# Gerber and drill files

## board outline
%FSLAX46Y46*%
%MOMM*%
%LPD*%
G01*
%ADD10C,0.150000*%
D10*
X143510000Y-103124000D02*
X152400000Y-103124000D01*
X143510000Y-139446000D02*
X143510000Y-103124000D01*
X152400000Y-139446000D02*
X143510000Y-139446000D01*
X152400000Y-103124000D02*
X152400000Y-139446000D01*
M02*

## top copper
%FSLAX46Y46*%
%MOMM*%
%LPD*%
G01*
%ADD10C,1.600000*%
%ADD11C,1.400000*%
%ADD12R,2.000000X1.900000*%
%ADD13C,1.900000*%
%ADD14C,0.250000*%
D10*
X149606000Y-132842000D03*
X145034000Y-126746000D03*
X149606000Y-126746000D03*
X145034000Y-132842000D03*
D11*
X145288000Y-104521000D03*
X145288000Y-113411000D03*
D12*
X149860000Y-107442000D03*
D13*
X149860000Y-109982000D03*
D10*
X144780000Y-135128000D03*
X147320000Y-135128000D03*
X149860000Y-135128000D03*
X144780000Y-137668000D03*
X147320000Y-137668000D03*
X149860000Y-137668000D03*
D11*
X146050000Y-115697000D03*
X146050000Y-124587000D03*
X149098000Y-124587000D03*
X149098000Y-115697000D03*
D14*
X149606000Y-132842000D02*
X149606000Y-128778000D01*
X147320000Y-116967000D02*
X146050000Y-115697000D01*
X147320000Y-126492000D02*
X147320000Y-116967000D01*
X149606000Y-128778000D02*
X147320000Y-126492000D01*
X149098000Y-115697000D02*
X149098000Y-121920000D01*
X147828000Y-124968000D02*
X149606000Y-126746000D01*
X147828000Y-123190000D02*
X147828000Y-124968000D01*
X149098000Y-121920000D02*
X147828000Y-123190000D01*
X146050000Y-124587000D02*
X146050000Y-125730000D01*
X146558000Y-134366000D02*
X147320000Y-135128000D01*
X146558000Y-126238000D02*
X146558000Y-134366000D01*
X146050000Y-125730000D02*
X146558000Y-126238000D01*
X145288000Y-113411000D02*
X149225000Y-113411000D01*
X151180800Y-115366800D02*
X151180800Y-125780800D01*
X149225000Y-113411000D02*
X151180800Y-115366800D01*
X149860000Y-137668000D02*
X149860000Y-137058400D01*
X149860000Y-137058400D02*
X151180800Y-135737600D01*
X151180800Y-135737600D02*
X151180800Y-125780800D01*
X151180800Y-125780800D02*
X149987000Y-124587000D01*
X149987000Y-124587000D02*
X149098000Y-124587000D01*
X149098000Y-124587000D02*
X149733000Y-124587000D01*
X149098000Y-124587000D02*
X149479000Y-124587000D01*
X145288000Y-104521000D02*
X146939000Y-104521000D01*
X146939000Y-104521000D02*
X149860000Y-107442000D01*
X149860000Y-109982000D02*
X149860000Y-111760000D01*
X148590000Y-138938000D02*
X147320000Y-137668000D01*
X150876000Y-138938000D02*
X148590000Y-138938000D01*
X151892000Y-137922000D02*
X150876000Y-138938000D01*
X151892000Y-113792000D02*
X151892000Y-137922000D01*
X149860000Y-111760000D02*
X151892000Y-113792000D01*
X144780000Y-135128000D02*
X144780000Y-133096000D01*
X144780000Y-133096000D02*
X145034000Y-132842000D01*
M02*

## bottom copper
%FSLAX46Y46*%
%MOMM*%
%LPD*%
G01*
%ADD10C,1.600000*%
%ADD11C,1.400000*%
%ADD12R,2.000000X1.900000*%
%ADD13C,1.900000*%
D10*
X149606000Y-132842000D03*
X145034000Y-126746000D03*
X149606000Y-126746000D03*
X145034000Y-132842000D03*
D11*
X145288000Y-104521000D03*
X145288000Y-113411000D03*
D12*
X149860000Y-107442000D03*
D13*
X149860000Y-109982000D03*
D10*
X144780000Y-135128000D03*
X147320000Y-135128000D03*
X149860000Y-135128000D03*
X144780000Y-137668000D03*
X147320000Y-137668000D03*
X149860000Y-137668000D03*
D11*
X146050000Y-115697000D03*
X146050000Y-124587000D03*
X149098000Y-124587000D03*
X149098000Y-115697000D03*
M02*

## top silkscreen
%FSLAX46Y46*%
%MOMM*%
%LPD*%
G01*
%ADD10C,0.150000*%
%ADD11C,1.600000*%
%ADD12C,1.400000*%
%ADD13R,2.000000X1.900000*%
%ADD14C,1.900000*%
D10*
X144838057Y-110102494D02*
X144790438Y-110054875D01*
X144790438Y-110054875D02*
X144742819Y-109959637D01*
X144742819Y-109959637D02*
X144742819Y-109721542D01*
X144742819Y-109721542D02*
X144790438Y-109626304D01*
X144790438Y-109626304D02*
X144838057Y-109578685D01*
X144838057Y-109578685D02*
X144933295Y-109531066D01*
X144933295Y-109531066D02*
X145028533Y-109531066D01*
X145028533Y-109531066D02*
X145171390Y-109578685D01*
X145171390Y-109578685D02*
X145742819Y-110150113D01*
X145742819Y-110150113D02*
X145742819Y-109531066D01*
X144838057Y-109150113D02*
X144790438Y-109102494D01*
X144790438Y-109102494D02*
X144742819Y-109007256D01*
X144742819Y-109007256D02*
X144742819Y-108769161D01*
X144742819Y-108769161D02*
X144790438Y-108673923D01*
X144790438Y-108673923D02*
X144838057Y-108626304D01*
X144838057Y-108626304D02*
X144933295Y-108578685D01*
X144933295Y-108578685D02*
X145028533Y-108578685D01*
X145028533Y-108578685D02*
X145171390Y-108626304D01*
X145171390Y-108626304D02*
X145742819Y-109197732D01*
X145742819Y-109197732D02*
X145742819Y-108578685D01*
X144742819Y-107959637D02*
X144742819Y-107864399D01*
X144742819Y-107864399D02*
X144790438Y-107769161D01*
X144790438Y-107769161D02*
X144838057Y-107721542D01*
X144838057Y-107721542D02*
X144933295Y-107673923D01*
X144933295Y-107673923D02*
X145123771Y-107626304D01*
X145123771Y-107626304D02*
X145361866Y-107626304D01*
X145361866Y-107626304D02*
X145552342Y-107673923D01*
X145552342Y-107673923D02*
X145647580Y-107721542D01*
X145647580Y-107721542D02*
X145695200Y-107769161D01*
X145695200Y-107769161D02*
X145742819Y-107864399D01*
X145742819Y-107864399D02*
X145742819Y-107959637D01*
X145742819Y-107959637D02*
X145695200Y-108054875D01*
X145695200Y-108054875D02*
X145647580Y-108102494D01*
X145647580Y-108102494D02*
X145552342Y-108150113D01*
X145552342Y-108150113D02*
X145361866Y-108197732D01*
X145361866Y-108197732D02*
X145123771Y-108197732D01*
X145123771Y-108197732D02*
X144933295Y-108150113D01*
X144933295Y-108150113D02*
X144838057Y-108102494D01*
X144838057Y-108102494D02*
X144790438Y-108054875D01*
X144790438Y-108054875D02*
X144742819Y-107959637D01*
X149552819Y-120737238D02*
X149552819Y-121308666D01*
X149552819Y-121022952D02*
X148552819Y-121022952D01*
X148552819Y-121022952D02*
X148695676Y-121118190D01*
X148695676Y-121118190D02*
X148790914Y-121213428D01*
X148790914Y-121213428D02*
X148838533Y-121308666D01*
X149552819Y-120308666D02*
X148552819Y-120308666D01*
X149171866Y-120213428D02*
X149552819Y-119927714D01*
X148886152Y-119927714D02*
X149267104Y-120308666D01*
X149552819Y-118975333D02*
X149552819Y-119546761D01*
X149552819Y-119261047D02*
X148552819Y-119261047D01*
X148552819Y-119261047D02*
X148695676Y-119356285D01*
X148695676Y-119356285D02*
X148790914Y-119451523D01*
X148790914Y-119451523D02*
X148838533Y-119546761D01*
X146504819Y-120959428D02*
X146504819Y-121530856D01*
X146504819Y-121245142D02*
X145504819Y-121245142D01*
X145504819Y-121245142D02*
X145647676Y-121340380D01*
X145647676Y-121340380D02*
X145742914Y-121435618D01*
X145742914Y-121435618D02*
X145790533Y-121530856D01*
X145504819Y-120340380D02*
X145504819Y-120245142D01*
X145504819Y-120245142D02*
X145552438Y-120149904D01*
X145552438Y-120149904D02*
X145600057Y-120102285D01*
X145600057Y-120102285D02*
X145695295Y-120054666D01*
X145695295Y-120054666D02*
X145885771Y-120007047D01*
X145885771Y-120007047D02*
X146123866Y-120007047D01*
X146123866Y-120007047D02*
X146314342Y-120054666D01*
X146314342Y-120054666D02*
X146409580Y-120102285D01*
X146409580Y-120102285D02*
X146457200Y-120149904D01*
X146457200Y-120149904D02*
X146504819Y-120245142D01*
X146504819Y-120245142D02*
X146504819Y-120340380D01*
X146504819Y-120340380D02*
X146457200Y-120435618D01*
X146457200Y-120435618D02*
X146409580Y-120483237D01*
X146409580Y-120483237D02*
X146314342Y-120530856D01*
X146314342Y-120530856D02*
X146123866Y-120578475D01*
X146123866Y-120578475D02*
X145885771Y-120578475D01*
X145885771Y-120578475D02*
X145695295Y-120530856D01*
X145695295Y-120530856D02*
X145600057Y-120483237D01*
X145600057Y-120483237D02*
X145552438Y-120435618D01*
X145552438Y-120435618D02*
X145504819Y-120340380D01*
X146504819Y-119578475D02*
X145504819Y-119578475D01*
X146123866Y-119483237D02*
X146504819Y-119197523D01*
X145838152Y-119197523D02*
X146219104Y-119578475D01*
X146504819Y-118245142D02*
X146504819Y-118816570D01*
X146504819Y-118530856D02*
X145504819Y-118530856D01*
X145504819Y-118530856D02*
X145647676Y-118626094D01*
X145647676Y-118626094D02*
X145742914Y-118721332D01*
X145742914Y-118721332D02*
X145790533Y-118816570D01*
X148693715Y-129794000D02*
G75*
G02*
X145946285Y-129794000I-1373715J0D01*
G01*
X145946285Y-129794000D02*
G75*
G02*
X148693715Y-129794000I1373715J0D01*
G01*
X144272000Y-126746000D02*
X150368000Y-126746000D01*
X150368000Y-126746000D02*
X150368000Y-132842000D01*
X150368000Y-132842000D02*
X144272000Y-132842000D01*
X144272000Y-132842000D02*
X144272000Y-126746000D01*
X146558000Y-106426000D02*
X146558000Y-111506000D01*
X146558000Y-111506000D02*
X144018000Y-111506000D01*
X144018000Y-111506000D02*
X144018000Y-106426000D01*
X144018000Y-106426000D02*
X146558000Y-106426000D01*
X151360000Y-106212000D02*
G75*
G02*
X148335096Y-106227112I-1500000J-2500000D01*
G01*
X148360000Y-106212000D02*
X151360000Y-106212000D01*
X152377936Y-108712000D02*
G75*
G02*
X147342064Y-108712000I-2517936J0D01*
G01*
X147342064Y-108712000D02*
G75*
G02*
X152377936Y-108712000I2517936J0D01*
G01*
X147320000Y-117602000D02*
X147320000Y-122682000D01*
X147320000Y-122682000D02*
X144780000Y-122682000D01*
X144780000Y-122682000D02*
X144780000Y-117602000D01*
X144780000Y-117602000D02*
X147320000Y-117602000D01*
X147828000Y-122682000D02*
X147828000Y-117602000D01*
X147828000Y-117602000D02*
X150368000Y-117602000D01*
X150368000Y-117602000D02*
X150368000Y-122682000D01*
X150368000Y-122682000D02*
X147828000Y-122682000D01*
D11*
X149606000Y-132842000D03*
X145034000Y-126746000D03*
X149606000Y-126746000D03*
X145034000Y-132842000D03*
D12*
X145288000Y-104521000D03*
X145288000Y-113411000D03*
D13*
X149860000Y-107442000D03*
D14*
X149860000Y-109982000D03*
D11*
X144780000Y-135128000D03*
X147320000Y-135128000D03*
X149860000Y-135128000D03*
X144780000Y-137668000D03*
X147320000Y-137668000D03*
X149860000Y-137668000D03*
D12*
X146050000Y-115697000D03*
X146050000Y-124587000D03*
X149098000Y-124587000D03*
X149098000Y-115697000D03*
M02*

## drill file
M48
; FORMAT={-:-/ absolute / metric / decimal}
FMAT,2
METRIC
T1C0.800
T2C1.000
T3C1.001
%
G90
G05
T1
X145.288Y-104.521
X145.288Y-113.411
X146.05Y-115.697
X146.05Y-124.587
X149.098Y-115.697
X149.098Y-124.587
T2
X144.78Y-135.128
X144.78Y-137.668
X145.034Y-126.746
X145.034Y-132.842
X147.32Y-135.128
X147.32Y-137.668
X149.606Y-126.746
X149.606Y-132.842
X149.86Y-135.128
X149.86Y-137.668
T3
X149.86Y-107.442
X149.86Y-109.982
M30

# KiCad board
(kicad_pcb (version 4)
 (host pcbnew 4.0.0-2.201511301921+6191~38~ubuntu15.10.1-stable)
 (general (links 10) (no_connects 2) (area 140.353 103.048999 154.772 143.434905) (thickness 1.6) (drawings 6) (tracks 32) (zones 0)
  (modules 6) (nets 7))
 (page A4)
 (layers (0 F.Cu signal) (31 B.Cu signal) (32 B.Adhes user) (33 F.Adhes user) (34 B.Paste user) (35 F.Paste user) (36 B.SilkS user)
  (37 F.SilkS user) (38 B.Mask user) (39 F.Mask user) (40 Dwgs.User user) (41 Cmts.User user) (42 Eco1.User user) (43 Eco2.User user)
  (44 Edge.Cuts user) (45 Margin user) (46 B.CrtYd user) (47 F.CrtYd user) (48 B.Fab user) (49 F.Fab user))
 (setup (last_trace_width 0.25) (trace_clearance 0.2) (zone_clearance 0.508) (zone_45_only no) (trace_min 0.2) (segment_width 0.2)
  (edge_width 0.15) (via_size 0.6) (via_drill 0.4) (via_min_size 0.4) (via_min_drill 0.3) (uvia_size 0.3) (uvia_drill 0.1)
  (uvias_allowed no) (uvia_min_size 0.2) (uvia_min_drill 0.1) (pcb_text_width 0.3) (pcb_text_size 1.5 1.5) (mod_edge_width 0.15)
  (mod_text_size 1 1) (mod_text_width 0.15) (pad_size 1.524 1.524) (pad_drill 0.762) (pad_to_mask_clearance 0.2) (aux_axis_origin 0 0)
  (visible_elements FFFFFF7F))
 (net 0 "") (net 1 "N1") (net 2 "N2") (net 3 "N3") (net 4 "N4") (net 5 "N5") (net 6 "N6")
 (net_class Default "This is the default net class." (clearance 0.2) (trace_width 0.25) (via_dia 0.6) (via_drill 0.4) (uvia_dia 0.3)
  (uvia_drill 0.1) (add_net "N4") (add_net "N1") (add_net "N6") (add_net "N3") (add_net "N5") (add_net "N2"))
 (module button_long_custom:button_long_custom (layer F.Cu) (at 147.32 129.794 180)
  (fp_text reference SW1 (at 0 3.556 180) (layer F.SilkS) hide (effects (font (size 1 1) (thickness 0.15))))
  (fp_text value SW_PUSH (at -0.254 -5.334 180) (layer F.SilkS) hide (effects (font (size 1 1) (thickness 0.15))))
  (fp_circle (center 0 0) (end -1.143 -0.762) (layer F.SilkS) (width 0.15))
  (fp_line (start 3.048 3.048) (end -3.048 3.048) (layer F.SilkS) (width 0.15))
  (fp_line (start -3.048 3.048) (end -3.048 -3.048) (layer F.SilkS) (width 0.15))
  (fp_line (start -3.048 -3.048) (end 3.048 -3.048) (layer F.SilkS) (width 0.15))
  (fp_line (start 3.048 -3.048) (end 3.048 3.048) (layer F.SilkS) (width 0.15))
  (pad 1 thru_hole circle (at -2.286 -3.048 180) (size 1.6 1.6) (drill 1) (layers *.Cu *.Mask F.SilkS) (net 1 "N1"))
  (pad 2 thru_hole circle (at 2.286 3.048 180) (size 1.6 1.6) (drill 1) (layers *.Cu *.Mask F.SilkS) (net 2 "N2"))
  (pad 1 thru_hole circle (at -2.286 3.048 180) (size 1.6 1.6) (drill 1) (layers *.Cu *.Mask F.SilkS) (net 1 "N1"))
  (pad 2 thru_hole circle (at 2.286 -3.048 180) (size 1.6 1.6) (drill 1) (layers *.Cu *.Mask F.SilkS) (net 2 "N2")))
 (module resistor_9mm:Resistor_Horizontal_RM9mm (layer F.Cu) (at 145.288 108.966 270)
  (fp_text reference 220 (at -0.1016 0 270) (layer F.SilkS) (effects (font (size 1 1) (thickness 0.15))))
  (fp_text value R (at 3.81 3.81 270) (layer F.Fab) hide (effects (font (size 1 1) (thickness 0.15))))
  (fp_line (start -2.54 -1.27) (end 2.54 -1.27) (layer F.SilkS) (width 0.15))
  (fp_line (start 2.54 -1.27) (end 2.54 1.27) (layer F.SilkS) (width 0.15))
  (fp_line (start 2.54 1.27) (end -2.54 1.27) (layer F.SilkS) (width 0.15))
  (fp_line (start -2.54 1.27) (end -2.54 -1.27) (layer F.SilkS) (width 0.15))
  (pad 1 thru_hole circle (at -4.445 0 270) (size 1.4 1.4) (drill 0.8) (layers *.Cu *.SilkS *.Mask) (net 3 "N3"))
  (pad 2 thru_hole circle (at 4.445 0 270) (size 1.4 1.4) (drill 0.8) (layers *.Cu *.SilkS *.Mask) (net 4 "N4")))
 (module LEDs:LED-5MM (layer F.Cu) (at 149.86 107.442 270)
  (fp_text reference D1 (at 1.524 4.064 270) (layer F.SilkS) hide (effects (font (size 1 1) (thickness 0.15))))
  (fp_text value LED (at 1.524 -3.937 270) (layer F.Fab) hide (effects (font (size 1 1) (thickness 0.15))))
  (fp_arc (start 1.27 0) (end -1.23 -1.5) (angle 297.5) (layer F.SilkS) (width 0.15))
  (fp_line (start -1.23 1.5) (end -1.23 -1.5) (layer F.SilkS) (width 0.15))
  (fp_circle (center 1.27 0) (end 0.97 -2.5) (layer F.SilkS) (width 0.15))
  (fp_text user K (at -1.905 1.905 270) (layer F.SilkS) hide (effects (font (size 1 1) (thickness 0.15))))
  (pad 1 thru_hole rect (at 0 0) (size 2 1.9) (drill 1.00076) (layers *.Cu *.Mask F.SilkS) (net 3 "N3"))
  (pad 2 thru_hole circle (at 2.54 0 270) (size 1.9 1.9) (drill 1.00076) (layers *.Cu *.Mask F.SilkS) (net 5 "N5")))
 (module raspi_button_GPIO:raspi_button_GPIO (layer F.Cu) (at 147.32 136.398)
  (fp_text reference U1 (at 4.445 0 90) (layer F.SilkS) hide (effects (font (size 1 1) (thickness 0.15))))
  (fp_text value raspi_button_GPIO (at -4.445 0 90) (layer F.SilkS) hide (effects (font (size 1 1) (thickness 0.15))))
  (pad 1 thru_hole circle (at -2.54 -1.27) (size 1.6 1.6) (drill 1) (layers *.Cu *.Mask F.SilkS) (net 2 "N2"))
  (pad 3 thru_hole circle (at 0 -1.27) (size 1.6 1.6) (drill 1) (layers *.Cu *.Mask F.SilkS) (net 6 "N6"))
  (pad 5 thru_hole circle (at 2.54 -1.27) (size 1.6 1.6) (drill 1) (layers *.Cu *.Mask F.SilkS))
  (pad 6 thru_hole circle (at -2.54 1.27) (size 1.6 1.6) (drill 1) (layers *.Cu *.Mask F.SilkS))
  (pad 4 thru_hole circle (at 0 1.27) (size 1.6 1.6) (drill 1) (layers *.Cu *.Mask F.SilkS) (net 5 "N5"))
  (pad 2 thru_hole circle (at 2.54 1.27) (size 1.6 1.6) (drill 1) (layers *.Cu *.Mask F.SilkS) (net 4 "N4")))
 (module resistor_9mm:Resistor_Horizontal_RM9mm (layer F.Cu) (at 146.05 120.142 270)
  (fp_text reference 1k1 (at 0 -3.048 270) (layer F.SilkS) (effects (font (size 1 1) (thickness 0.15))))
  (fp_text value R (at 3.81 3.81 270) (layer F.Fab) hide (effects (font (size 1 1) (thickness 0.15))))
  (fp_line (start -2.54 -1.27) (end 2.54 -1.27) (layer F.SilkS) (width 0.15))
  (fp_line (start 2.54 -1.27) (end 2.54 1.27) (layer F.SilkS) (width 0.15))
  (fp_line (start 2.54 1.27) (end -2.54 1.27) (layer F.SilkS) (width 0.15))
  (fp_line (start -2.54 1.27) (end -2.54 -1.27) (layer F.SilkS) (width 0.15))
  (pad 1 thru_hole circle (at -4.445 0 270) (size 1.4 1.4) (drill 0.8) (layers *.Cu *.SilkS *.Mask) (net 1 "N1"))
  (pad 2 thru_hole circle (at 4.445 0 270) (size 1.4 1.4) (drill 0.8) (layers *.Cu *.SilkS *.Mask) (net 6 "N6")))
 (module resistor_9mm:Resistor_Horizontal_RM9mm (layer F.Cu) (at 149.098 120.142 90)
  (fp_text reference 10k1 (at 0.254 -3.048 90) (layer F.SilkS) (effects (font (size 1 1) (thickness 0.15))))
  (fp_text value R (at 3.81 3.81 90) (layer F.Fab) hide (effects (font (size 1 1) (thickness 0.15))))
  (fp_line (start -2.54 -1.27) (end 2.54 -1.27) (layer F.SilkS) (width 0.15))
  (fp_line (start 2.54 -1.27) (end 2.54 1.27) (layer F.SilkS) (width 0.15))
  (fp_line (start 2.54 1.27) (end -2.54 1.27) (layer F.SilkS) (width 0.15))
  (fp_line (start -2.54 1.27) (end -2.54 -1.27) (layer F.SilkS) (width 0.15))
  (pad 1 thru_hole circle (at -4.445 0 90) (size 1.4 1.4) (drill 0.8) (layers *.Cu *.SilkS *.Mask) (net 4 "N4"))
  (pad 2 thru_hole circle (at 4.445 0 90) (size 1.4 1.4) (drill 0.8) (layers *.Cu *.SilkS *.Mask) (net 1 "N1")))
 (gr_line (start 143.51 103.124) (end 152.4 103.124) (angle 90) (layer Edge.Cuts) (width 0.15))
 (gr_line (start 143.51 139.446) (end 143.51 103.124) (angle 90) (layer Edge.Cuts) (width 0.15))
 (gr_line (start 152.4 139.446) (end 143.51 139.446) (angle 90) (layer Edge.Cuts) (width 0.15))
 (gr_line (start 152.4 103.124) (end 152.4 139.446) (angle 90) (layer Edge.Cuts) (width 0.15))
 (segment (start 149.606 132.842) (end 149.606 128.778) (width 0.25) (layer F.Cu) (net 1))
 (segment (start 147.32 116.967) (end 146.05 115.697) (width 0.25) (layer F.Cu) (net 1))
 (segment (start 147.32 126.492) (end 147.32 116.967) (width 0.25) (layer F.Cu) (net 1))
 (segment (start 149.606 128.778) (end 147.32 126.492) (width 0.25) (layer F.Cu) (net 1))
 (segment (start 149.098 115.697) (end 149.098 121.92) (width 0.25) (layer F.Cu) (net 1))
 (segment (start 147.828 124.968) (end 149.606 126.746) (width 0.25) (layer F.Cu) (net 1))
 (segment (start 147.828 123.19) (end 147.828 124.968) (width 0.25) (layer F.Cu) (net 1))
 (segment (start 149.098 121.92) (end 147.828 123.19) (width 0.25) (layer F.Cu) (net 1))
 (segment (start 146.05 124.587) (end 146.05 125.73) (width 0.25) (layer F.Cu) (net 6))
 (segment (start 146.558 134.366) (end 147.32 135.128) (width 0.25) (layer F.Cu) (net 6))
 (segment (start 146.558 126.238) (end 146.558 134.366) (width 0.25) (layer F.Cu) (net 6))
 (segment (start 146.05 125.73) (end 146.558 126.238) (width 0.25) (layer F.Cu) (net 6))
 (segment (start 145.288 113.411) (end 149.225 113.411) (width 0.25) (layer F.Cu) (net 4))
 (segment (start 151.1808 115.3668) (end 151.1808 125.7808) (width 0.25) (layer F.Cu) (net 4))
 (segment (start 149.225 113.411) (end 151.1808 115.3668) (width 0.25) (layer F.Cu) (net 4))
 (segment (start 149.86 137.668) (end 149.86 137.0584) (width 0.25) (layer F.Cu) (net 4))
 (segment (start 149.86 137.0584) (end 151.1808 135.7376) (width 0.25) (layer F.Cu) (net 4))
 (segment (start 151.1808 135.7376) (end 151.1808 125.7808) (width 0.25) (layer F.Cu) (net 4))
 (segment (start 151.1808 125.7808) (end 149.987 124.587) (width 0.25) (layer F.Cu) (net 4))
 (segment (start 149.987 124.587) (end 149.098 124.587) (width 0.25) (layer F.Cu) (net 4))
 (segment (start 149.098 124.587) (end 149.733 124.587) (width 0.25) (layer F.Cu) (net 4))
 (segment (start 149.098 124.587) (end 149.479 124.587) (width 0.25) (layer F.Cu) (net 4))
 (segment (start 145.288 104.521) (end 146.939 104.521) (width 0.25) (layer F.Cu) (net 3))
 (segment (start 146.939 104.521) (end 149.86 107.442) (width 0.25) (layer F.Cu) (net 3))
 (segment (start 149.86 109.982) (end 149.86 111.76) (width 0.25) (layer F.Cu) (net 5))
 (segment (start 148.59 138.938) (end 147.32 137.668) (width 0.25) (layer F.Cu) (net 5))
 (segment (start 150.876 138.938) (end 148.59 138.938) (width 0.25) (layer F.Cu) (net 5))
 (segment (start 151.892 137.922) (end 150.876 138.938) (width 0.25) (layer F.Cu) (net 5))
 (segment (start 151.892 113.792) (end 151.892 137.922) (width 0.25) (layer F.Cu) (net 5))
 (segment (start 149.86 111.76) (end 151.892 113.792) (width 0.25) (layer F.Cu) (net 5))
 (segment (start 144.78 135.128) (end 144.78 133.096) (width 0.25) (layer F.Cu) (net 2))
 (segment (start 144.78 133.096) (end 145.034 132.842) (width 0.25) (layer F.Cu) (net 2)))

